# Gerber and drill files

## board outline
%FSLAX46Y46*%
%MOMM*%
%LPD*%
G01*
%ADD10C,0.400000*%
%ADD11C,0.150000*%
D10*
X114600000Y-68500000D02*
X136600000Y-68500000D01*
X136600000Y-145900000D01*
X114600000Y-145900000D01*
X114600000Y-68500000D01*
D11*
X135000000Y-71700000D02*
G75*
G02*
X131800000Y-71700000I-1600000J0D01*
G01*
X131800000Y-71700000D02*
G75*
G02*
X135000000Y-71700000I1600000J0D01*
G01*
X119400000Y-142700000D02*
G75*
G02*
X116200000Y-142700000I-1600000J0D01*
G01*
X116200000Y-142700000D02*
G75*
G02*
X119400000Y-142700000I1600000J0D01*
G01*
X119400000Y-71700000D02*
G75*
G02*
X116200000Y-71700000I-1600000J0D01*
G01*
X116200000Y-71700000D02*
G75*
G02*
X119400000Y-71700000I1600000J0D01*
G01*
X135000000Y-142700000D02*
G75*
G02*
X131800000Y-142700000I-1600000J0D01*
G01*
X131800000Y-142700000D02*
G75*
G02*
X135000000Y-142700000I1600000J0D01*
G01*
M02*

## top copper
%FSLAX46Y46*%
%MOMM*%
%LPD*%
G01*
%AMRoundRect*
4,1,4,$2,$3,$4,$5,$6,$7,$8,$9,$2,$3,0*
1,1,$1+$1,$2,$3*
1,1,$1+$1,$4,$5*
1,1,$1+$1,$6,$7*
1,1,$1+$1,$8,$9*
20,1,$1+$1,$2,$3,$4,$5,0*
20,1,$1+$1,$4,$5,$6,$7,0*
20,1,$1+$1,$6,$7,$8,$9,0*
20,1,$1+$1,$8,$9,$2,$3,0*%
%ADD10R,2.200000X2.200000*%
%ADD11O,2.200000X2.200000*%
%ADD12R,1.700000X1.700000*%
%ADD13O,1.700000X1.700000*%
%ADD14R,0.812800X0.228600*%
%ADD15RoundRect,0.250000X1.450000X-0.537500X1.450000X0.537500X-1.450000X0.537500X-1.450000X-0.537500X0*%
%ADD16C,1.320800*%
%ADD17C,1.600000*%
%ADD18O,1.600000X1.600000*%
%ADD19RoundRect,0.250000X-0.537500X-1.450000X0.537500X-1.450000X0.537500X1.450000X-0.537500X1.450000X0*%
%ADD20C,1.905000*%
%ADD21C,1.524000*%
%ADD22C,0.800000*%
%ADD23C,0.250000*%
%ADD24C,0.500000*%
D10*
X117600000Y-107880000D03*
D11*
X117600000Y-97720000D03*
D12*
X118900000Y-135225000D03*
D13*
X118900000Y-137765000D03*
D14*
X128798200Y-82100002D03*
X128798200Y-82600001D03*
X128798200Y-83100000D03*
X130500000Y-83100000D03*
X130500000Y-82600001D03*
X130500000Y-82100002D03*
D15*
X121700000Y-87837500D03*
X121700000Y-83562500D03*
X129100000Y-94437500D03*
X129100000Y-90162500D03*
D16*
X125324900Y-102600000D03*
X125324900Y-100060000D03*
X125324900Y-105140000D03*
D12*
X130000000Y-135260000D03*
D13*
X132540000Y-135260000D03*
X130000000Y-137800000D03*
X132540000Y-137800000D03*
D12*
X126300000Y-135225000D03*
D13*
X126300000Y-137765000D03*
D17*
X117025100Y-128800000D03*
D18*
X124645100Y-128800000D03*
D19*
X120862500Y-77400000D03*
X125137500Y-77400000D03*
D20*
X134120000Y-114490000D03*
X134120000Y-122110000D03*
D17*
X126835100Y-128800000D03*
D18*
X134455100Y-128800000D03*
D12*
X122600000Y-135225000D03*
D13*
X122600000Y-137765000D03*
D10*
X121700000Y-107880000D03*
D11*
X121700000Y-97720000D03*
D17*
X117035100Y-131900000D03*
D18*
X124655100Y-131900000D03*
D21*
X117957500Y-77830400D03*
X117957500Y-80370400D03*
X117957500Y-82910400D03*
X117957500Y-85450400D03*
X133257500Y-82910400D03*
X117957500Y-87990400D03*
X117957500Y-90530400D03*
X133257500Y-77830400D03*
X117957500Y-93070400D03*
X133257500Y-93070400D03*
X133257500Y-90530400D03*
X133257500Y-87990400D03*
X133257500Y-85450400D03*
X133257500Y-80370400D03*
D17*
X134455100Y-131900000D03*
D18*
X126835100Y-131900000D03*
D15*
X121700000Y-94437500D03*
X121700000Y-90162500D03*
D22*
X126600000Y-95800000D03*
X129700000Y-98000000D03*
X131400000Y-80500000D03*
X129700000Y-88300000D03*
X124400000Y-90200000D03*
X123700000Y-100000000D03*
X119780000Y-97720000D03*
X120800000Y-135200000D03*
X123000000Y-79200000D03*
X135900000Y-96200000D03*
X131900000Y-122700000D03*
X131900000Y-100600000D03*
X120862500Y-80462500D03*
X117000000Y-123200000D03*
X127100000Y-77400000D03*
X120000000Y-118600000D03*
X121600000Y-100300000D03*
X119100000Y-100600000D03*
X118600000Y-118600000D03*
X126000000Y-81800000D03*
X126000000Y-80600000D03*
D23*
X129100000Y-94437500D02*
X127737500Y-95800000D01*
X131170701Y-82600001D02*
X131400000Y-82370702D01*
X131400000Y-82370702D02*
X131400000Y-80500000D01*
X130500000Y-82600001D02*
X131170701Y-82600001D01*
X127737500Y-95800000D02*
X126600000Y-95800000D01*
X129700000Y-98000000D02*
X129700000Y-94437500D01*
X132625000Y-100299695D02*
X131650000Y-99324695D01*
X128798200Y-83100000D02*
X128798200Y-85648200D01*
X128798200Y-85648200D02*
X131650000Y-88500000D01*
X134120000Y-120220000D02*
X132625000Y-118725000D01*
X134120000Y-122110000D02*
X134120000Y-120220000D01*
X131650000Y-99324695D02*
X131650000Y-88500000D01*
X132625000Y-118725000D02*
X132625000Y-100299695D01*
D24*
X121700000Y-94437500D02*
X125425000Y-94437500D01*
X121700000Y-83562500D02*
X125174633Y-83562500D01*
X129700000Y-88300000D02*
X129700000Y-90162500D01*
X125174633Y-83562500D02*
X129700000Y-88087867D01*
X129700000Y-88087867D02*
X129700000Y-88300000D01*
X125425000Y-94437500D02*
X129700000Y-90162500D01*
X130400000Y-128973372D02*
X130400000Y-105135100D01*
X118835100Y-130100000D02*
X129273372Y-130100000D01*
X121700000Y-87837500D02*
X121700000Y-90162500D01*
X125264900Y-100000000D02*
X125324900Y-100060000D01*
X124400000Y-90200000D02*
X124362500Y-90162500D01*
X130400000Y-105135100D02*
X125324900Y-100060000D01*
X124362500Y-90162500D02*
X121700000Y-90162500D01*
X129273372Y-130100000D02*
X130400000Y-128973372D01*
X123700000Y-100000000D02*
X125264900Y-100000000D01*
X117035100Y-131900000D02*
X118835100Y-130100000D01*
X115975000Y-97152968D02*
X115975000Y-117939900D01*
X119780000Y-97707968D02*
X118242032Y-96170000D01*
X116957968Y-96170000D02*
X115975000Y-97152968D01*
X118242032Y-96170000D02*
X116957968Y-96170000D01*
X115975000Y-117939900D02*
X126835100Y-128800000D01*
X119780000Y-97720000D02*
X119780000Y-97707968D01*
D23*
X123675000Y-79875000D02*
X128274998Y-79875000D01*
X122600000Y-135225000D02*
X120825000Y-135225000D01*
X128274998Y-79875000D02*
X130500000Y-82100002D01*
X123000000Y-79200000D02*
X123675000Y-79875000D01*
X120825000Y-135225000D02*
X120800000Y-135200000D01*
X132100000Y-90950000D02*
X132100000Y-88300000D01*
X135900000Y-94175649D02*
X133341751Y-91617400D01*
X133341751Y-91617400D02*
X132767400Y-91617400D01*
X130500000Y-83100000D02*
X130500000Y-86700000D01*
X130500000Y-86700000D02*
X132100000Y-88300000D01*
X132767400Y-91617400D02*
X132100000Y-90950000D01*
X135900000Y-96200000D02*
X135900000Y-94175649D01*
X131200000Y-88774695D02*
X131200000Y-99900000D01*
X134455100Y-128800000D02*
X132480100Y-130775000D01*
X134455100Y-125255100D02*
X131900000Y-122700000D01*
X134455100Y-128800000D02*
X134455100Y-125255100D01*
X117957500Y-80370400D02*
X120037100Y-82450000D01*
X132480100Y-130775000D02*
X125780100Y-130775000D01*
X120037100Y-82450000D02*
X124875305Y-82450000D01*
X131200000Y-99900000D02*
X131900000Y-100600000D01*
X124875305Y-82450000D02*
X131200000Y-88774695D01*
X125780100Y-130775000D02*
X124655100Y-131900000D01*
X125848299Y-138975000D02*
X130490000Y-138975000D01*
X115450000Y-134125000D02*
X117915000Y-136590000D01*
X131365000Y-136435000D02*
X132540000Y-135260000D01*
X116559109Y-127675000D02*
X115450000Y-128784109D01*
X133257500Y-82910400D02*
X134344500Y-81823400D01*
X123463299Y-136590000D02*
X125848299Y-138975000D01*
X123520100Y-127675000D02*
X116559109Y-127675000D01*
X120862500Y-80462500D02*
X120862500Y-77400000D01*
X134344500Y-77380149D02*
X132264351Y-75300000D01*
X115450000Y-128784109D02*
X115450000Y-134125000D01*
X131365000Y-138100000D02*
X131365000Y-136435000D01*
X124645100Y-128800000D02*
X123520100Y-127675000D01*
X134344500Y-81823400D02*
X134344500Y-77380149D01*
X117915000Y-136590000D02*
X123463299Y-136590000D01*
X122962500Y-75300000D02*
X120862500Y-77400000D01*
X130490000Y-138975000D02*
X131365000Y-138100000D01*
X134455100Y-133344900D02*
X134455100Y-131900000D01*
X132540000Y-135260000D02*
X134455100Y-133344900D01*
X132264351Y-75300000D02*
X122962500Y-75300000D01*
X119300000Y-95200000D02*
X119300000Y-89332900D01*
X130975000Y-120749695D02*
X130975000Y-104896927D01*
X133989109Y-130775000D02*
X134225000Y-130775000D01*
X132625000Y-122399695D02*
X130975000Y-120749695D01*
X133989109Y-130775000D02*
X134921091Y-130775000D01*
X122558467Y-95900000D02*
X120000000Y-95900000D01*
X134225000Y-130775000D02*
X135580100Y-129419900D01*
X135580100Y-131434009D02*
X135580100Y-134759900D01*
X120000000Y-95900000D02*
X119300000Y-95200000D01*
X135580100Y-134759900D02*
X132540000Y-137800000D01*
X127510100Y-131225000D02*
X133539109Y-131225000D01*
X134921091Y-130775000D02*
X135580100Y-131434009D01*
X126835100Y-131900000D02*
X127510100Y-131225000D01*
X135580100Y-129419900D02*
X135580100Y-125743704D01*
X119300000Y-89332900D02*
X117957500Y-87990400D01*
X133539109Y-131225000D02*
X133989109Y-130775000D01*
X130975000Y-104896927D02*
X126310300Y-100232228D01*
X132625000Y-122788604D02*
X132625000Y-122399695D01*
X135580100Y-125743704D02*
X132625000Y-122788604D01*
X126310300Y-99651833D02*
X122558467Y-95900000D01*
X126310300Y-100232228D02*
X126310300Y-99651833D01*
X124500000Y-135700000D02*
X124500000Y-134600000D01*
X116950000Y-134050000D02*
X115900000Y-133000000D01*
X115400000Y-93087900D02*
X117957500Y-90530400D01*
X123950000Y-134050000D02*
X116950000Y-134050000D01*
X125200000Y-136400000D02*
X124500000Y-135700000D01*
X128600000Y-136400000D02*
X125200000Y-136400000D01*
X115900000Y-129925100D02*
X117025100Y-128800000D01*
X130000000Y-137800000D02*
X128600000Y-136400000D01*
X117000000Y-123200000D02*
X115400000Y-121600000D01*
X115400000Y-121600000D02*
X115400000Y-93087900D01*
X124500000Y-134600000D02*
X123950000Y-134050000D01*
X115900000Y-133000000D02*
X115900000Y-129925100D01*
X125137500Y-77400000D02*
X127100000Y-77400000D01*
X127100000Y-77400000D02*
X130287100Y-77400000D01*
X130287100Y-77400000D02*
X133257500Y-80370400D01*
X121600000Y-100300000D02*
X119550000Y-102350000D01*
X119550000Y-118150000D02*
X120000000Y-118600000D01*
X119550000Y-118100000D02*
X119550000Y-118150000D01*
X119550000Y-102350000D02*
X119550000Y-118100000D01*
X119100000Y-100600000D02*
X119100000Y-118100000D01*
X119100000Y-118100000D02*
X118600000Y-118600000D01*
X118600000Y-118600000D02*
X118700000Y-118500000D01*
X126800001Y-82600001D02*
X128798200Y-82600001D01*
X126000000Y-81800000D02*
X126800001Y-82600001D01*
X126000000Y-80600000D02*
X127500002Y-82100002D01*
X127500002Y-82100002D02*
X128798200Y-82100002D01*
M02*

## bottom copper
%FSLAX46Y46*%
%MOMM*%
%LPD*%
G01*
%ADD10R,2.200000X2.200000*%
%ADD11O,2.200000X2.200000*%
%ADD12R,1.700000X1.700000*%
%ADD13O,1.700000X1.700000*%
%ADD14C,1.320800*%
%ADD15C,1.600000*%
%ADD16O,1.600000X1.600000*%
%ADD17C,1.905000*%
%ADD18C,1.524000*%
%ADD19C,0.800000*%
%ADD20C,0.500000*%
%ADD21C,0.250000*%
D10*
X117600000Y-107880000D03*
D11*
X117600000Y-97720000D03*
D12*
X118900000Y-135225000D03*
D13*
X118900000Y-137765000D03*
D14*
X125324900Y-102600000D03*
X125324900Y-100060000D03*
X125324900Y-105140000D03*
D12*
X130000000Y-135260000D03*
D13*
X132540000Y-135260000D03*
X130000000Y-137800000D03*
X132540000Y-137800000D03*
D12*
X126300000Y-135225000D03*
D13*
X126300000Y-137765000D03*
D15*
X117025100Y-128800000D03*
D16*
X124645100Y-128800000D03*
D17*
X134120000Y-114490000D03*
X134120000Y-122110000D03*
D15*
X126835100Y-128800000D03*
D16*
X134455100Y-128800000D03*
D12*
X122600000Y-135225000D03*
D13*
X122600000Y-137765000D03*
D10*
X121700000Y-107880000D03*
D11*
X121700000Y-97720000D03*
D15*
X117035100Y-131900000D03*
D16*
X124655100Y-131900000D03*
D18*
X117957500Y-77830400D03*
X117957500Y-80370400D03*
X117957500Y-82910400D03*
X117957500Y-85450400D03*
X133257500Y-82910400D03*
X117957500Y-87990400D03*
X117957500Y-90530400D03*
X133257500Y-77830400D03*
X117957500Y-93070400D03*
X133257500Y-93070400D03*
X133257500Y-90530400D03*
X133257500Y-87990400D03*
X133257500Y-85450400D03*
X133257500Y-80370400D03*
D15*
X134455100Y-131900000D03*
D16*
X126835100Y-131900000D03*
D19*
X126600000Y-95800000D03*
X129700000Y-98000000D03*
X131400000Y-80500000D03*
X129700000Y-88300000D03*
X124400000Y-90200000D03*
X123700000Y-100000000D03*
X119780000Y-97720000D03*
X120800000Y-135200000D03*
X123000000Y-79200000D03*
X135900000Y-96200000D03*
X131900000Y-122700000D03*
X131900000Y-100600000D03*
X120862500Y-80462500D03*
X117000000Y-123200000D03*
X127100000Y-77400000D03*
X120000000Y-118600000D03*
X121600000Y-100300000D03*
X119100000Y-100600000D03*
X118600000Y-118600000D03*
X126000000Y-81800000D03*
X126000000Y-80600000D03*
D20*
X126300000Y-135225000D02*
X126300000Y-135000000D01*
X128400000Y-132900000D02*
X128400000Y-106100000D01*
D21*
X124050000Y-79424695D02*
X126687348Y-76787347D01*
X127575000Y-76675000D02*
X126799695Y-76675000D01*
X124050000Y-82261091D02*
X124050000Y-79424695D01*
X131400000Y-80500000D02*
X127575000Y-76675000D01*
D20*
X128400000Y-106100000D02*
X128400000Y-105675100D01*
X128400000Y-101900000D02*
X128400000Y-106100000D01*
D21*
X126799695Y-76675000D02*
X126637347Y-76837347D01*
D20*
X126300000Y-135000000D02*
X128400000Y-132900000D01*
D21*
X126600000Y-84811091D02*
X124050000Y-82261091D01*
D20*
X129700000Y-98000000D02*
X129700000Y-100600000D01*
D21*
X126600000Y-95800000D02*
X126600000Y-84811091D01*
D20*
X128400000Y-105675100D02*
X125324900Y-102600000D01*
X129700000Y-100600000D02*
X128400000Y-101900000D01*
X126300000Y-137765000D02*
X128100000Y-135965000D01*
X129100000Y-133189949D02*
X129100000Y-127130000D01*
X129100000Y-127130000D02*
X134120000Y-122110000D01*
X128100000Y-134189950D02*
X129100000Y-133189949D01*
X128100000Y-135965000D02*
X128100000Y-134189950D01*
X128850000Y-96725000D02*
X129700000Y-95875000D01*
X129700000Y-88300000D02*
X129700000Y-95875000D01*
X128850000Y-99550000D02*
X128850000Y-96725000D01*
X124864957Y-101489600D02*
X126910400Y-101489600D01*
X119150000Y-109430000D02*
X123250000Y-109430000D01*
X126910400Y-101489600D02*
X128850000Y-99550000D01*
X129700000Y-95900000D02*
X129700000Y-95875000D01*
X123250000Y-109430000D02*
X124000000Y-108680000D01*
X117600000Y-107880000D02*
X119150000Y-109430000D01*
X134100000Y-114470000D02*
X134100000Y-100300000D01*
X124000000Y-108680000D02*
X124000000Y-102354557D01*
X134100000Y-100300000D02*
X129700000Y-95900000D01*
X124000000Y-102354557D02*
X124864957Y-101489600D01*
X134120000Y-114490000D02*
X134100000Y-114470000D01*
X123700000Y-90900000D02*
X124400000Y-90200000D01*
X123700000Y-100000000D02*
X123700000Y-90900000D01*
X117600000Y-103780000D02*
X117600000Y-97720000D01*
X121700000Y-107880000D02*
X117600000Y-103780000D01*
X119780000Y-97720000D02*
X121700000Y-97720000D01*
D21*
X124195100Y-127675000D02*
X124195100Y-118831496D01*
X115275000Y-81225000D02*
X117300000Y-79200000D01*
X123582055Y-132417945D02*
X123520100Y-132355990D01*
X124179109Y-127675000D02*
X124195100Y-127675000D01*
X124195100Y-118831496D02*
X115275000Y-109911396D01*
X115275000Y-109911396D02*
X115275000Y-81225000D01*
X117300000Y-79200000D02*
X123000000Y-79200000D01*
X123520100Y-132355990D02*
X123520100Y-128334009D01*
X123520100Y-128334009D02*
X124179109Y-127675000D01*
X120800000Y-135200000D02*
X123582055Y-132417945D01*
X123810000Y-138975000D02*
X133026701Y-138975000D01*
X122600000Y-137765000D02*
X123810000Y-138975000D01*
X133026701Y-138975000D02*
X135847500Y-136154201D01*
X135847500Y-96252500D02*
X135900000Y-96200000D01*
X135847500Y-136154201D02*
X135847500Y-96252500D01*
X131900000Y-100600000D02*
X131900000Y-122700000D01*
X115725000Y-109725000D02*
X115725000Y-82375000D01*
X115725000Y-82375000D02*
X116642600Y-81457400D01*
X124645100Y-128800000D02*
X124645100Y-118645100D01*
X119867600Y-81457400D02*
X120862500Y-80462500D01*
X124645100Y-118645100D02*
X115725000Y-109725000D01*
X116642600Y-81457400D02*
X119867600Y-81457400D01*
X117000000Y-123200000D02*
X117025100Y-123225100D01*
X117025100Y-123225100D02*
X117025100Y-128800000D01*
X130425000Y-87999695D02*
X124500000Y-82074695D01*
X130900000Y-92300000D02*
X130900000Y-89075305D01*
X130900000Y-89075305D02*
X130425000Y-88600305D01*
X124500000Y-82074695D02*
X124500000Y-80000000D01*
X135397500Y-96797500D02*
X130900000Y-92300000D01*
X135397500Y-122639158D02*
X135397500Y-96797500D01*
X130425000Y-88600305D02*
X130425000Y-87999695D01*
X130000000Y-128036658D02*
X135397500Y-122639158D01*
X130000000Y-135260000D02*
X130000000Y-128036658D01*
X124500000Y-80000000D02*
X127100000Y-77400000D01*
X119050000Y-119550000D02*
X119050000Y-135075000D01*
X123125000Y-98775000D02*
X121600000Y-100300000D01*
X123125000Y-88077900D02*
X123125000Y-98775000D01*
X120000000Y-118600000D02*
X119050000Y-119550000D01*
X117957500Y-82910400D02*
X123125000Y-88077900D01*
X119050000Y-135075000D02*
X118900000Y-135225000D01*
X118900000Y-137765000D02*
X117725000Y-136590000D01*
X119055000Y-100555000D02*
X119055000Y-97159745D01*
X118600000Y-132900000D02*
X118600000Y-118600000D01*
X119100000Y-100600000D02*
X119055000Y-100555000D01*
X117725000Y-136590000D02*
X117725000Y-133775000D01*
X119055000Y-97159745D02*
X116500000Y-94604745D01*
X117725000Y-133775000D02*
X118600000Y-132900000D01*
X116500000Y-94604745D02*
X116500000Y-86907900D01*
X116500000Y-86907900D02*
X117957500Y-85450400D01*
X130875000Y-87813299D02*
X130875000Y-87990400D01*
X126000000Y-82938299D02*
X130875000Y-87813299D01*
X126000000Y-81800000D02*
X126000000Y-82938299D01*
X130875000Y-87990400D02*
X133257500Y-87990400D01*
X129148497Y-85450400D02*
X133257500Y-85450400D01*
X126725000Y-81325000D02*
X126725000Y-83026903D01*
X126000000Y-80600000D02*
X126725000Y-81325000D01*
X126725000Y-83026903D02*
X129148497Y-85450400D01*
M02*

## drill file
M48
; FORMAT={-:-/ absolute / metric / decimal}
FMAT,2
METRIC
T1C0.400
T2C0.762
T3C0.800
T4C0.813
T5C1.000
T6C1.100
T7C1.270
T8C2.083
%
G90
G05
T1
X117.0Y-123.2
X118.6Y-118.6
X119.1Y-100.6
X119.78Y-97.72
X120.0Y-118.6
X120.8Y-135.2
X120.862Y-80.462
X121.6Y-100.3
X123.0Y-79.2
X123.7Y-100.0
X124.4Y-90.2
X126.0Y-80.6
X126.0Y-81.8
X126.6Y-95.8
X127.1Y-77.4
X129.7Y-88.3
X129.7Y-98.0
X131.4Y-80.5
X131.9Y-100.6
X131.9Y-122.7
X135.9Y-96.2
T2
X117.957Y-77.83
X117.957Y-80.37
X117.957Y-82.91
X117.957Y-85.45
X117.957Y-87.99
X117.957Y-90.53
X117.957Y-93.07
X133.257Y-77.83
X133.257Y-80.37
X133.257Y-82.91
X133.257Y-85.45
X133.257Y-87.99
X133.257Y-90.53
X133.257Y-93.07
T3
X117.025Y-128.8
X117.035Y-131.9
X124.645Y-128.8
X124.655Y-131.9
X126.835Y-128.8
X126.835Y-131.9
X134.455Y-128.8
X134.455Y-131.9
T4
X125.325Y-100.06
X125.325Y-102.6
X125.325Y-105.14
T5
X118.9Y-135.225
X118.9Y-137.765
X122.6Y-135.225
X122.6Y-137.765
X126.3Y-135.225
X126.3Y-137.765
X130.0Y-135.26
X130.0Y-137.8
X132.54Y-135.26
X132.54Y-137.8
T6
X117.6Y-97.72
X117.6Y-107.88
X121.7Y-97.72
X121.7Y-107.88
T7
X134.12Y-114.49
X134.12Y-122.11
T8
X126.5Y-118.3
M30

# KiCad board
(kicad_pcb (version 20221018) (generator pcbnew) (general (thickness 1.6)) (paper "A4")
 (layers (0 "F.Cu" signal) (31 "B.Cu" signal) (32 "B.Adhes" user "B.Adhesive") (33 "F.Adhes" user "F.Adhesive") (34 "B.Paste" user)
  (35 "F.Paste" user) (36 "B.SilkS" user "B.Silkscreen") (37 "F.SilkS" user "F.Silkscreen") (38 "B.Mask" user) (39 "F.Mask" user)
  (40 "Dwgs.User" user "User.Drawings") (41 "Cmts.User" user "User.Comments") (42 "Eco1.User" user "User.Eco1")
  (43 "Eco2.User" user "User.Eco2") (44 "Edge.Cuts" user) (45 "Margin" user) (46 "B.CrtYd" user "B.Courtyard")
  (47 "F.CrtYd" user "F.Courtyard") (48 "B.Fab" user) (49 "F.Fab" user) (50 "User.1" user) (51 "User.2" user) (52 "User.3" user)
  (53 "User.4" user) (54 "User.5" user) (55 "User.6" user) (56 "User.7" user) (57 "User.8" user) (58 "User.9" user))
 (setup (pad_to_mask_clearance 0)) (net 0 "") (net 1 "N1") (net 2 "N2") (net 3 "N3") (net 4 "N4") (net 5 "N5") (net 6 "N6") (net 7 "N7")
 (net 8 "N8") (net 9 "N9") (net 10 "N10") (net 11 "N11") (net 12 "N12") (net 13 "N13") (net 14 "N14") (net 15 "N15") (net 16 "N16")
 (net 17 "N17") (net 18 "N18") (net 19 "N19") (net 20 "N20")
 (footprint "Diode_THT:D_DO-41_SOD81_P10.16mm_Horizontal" (layer "F.Cu") (at 117.6 107.88 90)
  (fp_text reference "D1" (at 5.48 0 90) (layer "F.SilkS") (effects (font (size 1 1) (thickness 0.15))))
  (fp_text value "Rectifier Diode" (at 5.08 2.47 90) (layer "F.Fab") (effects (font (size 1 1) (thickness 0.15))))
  (pad "1" thru_hole rect (at 0 0 90) (size 2.2 2.2) (drill 1.1) (layers "*.Cu" "*.Mask") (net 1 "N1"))
  (pad "2" thru_hole oval (at 10.16 0 90) (size 2.2 2.2) (drill 1.1) (layers "*.Cu" "*.Mask") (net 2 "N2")))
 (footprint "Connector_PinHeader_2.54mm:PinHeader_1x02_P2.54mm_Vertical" (layer "F.Cu") (at 118.9 135.225)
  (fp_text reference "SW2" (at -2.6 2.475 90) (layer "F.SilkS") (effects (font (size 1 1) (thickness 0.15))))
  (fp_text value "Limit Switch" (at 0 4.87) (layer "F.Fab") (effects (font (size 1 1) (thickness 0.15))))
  (pad "1" thru_hole rect (at 0 0) (size 1.7 1.7) (drill 1) (layers "*.Cu" "*.Mask") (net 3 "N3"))
  (pad "2" thru_hole oval (at 0 2.54) (size 1.7 1.7) (drill 1) (layers "*.Cu" "*.Mask") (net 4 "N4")))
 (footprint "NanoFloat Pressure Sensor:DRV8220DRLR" (layer "F.Cu") (at 129.6491 82.600001)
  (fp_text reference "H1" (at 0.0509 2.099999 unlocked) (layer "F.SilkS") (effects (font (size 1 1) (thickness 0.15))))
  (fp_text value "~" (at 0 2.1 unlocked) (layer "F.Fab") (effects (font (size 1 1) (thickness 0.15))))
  (pad "1" smd rect (at -0.8509 -0.499999) (size 0.8128 0.2286) (layers "F.Cu" "F.Paste" "F.Mask") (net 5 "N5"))
  (pad "2" smd rect (at -0.8509 0) (size 0.8128 0.2286) (layers "F.Cu" "F.Paste" "F.Mask") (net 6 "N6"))
  (pad "3" smd rect (at -0.8509 0.499999) (size 0.8128 0.2286) (layers "F.Cu" "F.Paste" "F.Mask") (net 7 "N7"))
  (pad "4" smd rect (at 0.8509 0.499999) (size 0.8128 0.2286) (layers "F.Cu" "F.Paste" "F.Mask") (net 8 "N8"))
  (pad "5" smd rect (at 0.8509 0) (size 0.8128 0.2286) (layers "F.Cu" "F.Paste" "F.Mask") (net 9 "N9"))
  (pad "6" smd rect (at 0.8509 -0.499999) (size 0.8128 0.2286) (layers "F.Cu" "F.Paste" "F.Mask") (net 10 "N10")))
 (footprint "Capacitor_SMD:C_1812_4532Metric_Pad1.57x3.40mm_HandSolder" (layer "F.Cu") (at 121.7 85.7 90)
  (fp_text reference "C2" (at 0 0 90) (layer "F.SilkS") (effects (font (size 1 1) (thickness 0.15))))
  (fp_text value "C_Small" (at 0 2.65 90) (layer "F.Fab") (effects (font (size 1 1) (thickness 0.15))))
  (pad "1" smd roundrect (at -2.1375 0 90) (size 1.575 3.4) (layers "F.Cu" "F.Paste" "F.Mask") (roundrect_rratio 0.1587301587)
   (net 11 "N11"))
  (pad "2" smd roundrect (at 2.1375 0 90) (size 1.575 3.4) (layers "F.Cu" "F.Paste" "F.Mask") (roundrect_rratio 0.1587301587) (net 1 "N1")))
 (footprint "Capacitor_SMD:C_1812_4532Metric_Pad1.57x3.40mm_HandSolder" (layer "F.Cu") (at 129.1 92.3 90)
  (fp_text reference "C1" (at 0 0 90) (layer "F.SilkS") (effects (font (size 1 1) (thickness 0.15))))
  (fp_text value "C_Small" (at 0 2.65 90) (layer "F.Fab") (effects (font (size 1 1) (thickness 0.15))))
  (pad "1" smd roundrect (at -2.1375 0 90) (size 1.575 3.4) (layers "F.Cu" "F.Paste" "F.Mask") (roundrect_rratio 0.1587301587) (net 9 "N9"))
  (pad "2" smd roundrect (at 2.1375 0 90) (size 1.575 3.4) (layers "F.Cu" "F.Paste" "F.Mask") (roundrect_rratio 0.1587301587) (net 1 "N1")))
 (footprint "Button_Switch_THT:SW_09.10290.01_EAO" (layer "F.Cu") (at 125.3249 102.6 90)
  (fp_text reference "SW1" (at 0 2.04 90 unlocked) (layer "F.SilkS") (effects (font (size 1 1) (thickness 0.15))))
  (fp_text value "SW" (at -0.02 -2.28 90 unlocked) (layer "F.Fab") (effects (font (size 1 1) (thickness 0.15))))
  (pad "1" thru_hole circle (at 0 0 90) (size 1.3208 1.3208) (drill 0.8128) (layers "*.Cu" "*.Mask") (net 9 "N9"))
  (pad "2" thru_hole circle (at 2.54 0 90) (size 1.3208 1.3208) (drill 0.8128) (layers "*.Cu" "*.Mask") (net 11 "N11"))
  (pad "3" thru_hole circle (at -2.54 0 90) (size 1.3208 1.3208) (drill 0.8128) (layers "*.Cu" "*.Mask") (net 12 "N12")))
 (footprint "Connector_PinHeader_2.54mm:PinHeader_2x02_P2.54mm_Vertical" (layer "F.Cu") (at 130 135.26)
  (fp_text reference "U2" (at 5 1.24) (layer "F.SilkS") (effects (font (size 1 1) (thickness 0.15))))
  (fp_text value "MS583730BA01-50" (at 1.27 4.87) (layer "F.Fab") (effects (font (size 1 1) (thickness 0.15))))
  (pad "1" thru_hole rect (at 0 0) (size 1.7 1.7) (drill 1) (layers "*.Cu" "*.Mask") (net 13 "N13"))
  (pad "2" thru_hole oval (at 2.54 0) (size 1.7 1.7) (drill 1) (layers "*.Cu" "*.Mask") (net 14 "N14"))
  (pad "3" thru_hole oval (at 0 2.54) (size 1.7 1.7) (drill 1) (layers "*.Cu" "*.Mask") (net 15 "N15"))
  (pad "4" thru_hole oval (at 2.54 2.54) (size 1.7 1.7) (drill 1) (layers "*.Cu" "*.Mask") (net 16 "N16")))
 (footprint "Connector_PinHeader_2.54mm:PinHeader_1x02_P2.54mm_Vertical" (layer "F.Cu") (at 126.3 135.225)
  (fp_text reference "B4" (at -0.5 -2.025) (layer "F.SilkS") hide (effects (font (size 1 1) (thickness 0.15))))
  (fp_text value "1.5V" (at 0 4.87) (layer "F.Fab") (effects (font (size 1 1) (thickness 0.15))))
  (pad "1" thru_hole rect (at 0 0) (size 1.7 1.7) (drill 1) (layers "*.Cu" "*.Mask") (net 9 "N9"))
  (pad "2" thru_hole oval (at 0 2.54) (size 1.7 1.7) (drill 1) (layers "*.Cu" "*.Mask") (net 7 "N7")))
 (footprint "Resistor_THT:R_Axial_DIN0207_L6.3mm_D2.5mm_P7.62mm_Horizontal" (layer "F.Cu") (at 117.0251 128.8)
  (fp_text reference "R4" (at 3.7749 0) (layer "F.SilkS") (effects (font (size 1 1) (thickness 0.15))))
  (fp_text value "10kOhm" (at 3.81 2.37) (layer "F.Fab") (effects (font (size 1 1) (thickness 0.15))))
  (pad "1" thru_hole circle (at 0 0) (size 1.6 1.6) (drill 0.8) (layers "*.Cu" "*.Mask") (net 15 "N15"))
  (pad "2" thru_hole oval (at 7.62 0) (size 1.6 1.6) (drill 0.8) (layers "*.Cu" "*.Mask") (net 14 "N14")))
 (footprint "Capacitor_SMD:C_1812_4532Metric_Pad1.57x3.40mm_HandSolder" (layer "F.Cu") (at 123 77.4)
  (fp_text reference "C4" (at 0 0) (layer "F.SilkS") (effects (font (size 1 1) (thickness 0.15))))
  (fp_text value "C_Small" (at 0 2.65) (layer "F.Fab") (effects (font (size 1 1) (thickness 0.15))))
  (pad "1" smd roundrect (at -2.1375 0) (size 1.575 3.4) (layers "F.Cu" "F.Paste" "F.Mask") (roundrect_rratio 0.1587301587) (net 14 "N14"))
  (pad "2" smd roundrect (at 2.1375 0) (size 1.575 3.4) (layers "F.Cu" "F.Paste" "F.Mask") (roundrect_rratio 0.1587301587) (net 13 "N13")))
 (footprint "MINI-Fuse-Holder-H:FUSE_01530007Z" (layer "F.Cu") (at 126.5 118.3 -90)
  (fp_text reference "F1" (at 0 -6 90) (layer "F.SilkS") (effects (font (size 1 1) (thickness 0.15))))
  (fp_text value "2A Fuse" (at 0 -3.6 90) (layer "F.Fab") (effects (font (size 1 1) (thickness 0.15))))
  (pad "" np_thru_hole circle (at 0 0 270) (size 2.0828 2.0828) (drill 2.0828) (layers "*.Cu" "*.Mask"))
  (pad "1" thru_hole circle (at -3.81 -7.62 270) (size 1.905 1.905) (drill 1.27) (layers "*.Cu" "*.Mask") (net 1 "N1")
   (solder_mask_margin 0.102))
  (pad "2" thru_hole circle (at 3.81 -7.62 270) (size 1.905 1.905) (drill 1.27) (layers "*.Cu" "*.Mask") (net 7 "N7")
   (solder_mask_margin 0.102)))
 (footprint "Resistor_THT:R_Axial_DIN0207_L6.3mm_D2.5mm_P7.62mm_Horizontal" (layer "F.Cu") (at 126.8351 128.8)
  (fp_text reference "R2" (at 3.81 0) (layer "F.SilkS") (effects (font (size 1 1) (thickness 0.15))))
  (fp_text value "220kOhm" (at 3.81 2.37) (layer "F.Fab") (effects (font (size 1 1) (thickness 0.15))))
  (pad "1" thru_hole circle (at 0 0) (size 1.6 1.6) (drill 0.8) (layers "*.Cu" "*.Mask") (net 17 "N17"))
  (pad "2" thru_hole oval (at 7.62 0) (size 1.6 1.6) (drill 0.8) (layers "*.Cu" "*.Mask") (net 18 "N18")))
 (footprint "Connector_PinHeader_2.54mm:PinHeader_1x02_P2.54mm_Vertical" (layer "F.Cu") (at 122.6 135.225)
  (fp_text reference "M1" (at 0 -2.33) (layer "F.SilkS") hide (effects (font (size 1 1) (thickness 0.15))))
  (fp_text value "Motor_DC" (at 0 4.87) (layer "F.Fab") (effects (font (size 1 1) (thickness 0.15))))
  (pad "1" thru_hole rect (at 0 0) (size 1.7 1.7) (drill 1) (layers "*.Cu" "*.Mask") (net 10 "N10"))
  (pad "2" thru_hole oval (at 0 2.54) (size 1.7 1.7) (drill 1) (layers "*.Cu" "*.Mask") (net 8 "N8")))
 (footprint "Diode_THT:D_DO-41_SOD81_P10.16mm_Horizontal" (layer "F.Cu") (at 121.7 107.88 90)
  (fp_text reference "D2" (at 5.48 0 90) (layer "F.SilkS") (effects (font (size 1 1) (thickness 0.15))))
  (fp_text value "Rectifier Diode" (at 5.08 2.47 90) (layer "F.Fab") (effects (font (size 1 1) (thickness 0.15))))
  (pad "1" thru_hole rect (at 0 0 90) (size 2.2 2.2) (drill 1.1) (layers "*.Cu" "*.Mask") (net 2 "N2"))
  (pad "2" thru_hole oval (at 10.16 0 90) (size 2.2 2.2) (drill 1.1) (layers "*.Cu" "*.Mask") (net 17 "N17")))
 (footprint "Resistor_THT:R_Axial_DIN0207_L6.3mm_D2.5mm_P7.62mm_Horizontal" (layer "F.Cu") (at 117.0351 131.9)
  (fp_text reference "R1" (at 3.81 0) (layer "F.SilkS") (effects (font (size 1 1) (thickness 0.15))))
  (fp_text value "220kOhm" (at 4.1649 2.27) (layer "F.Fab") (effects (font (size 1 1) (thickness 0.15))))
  (pad "1" thru_hole circle (at 0 0) (size 1.6 1.6) (drill 0.8) (layers "*.Cu" "*.Mask") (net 11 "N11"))
  (pad "2" thru_hole oval (at 7.62 0) (size 1.6 1.6) (drill 0.8) (layers "*.Cu" "*.Mask") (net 18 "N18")))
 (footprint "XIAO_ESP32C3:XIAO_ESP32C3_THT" (layer "F.Cu") (at 125.5575 87.8704)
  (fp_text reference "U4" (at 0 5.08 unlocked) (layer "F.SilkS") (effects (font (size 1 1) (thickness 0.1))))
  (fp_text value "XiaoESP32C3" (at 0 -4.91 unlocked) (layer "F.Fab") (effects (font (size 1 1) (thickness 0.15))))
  (pad "0" thru_hole circle (at -7.6 -10.04) (size 1.524 1.524) (drill 0.762) (layers "*.Cu" "*.Mask"))
  (pad "1" thru_hole circle (at -7.6 -7.5) (size 1.524 1.524) (drill 0.762) (layers "*.Cu" "*.Mask") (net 18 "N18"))
  (pad "2" thru_hole circle (at -7.6 -4.96) (size 1.524 1.524) (drill 0.762) (layers "*.Cu" "*.Mask") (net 3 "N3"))
  (pad "3" thru_hole circle (at -7.6 -2.42) (size 1.524 1.524) (drill 0.762) (layers "*.Cu" "*.Mask") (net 4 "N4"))
  (pad "3V3" thru_hole circle (at 7.7 -4.96) (size 1.524 1.524) (drill 0.762) (layers "*.Cu" "*.Mask") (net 14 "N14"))
  (pad "4" thru_hole circle (at -7.6 0.12) (size 1.524 1.524) (drill 0.762) (layers "*.Cu" "*.Mask") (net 16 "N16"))
  (pad "5" thru_hole circle (at -7.6 2.66) (size 1.524 1.524) (drill 0.762) (layers "*.Cu" "*.Mask") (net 15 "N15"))
  (pad "5V" thru_hole circle (at 7.7 -10.04) (size 1.524 1.524) (drill 0.762) (layers "*.Cu" "*.Mask"))
  (pad "6" thru_hole circle (at -7.6 5.2) (size 1.524 1.524) (drill 0.762) (layers "*.Cu" "*.Mask"))
  (pad "7" thru_hole circle (at 7.7 5.2) (size 1.524 1.524) (drill 0.762) (layers "*.Cu" "*.Mask") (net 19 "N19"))
  (pad "8" thru_hole circle (at 7.7 2.66) (size 1.524 1.524) (drill 0.762) (layers "*.Cu" "*.Mask") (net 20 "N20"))
  (pad "9" thru_hole circle (at 7.7 0.12) (size 1.524 1.524) (drill 0.762) (layers "*.Cu" "*.Mask") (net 6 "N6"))
  (pad "10" thru_hole circle (at 7.7 -2.42) (size 1.524 1.524) (drill 0.762) (layers "*.Cu" "*.Mask") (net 5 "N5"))
  (pad "GND" thru_hole circle (at 7.7 -7.5) (size 1.524 1.524) (drill 0.762) (layers "*.Cu" "*.Mask") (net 13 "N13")))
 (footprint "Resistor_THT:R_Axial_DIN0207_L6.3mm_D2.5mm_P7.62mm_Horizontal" (layer "F.Cu") (at 134.4551 131.9 180)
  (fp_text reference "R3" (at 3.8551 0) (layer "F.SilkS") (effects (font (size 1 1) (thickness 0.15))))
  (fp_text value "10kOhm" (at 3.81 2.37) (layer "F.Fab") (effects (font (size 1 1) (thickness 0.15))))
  (pad "1" thru_hole circle (at 0 0 180) (size 1.6 1.6) (drill 0.8) (layers "*.Cu" "*.Mask") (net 14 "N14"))
  (pad "2" thru_hole oval (at 7.62 0 180) (size 1.6 1.6) (drill 0.8) (layers "*.Cu" "*.Mask") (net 16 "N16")))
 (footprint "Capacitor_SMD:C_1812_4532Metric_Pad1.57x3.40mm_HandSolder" (layer "F.Cu") (at 121.7 92.3 90)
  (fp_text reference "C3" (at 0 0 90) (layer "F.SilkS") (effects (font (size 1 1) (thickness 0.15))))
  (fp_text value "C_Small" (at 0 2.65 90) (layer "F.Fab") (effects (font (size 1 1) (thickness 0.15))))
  (pad "1" smd roundrect (at -2.1375 0 90) (size 1.575 3.4) (layers "F.Cu" "F.Paste" "F.Mask") (roundrect_rratio 0.1587301587) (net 1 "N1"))
  (pad "2" smd roundrect (at 2.1375 0 90) (size 1.575 3.4) (layers "F.Cu" "F.Paste" "F.Mask") (roundrect_rratio 0.1587301587) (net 11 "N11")))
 (gr_rect (start 114.6 68.5) (end 136.6 145.9) (stroke (width 0.4) (type default)) (fill none) (layer "Edge.Cuts"))
 (gr_circle (center 133.4 71.7) (end 135 71.7) (stroke (width 0.15) (type default)) (fill none) (layer "Edge.Cuts"))
 (gr_circle (center 117.8 142.7) (end 119.4 142.7) (stroke (width 0.15) (type default)) (fill none) (layer "Edge.Cuts"))
 (gr_circle (center 117.8 71.7) (end 119.4 71.7) (stroke (width 0.15) (type default)) (fill none) (layer "Edge.Cuts"))
 (gr_circle (center 133.4 142.7) (end 135 142.7) (stroke (width 0.15) (type default)) (fill none) (layer "Edge.Cuts"))
 (segment (start 129.1 94.4375) (end 127.7375 95.8) (width 0.25) (layer "F.Cu") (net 9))
 (segment (start 131.170701 82.600001) (end 131.4 82.370702) (width 0.25) (layer "F.Cu") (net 9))
 (segment (start 131.4 82.370702) (end 131.4 80.5) (width 0.25) (layer "F.Cu") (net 9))
 (segment (start 130.5 82.600001) (end 131.170701 82.600001) (width 0.25) (layer "F.Cu") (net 9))
 (segment (start 127.7375 95.8) (end 126.6 95.8) (width 0.25) (layer "F.Cu") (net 9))
 (segment (start 129.7 98) (end 129.7 94.4375) (width 0.25) (layer "F.Cu") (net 9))
 (via (at 126.6 95.8) (size 0.8) (drill 0.4) (layers "F.Cu" "B.Cu") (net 9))
 (via (at 129.7 98) (size 0.8) (drill 0.4) (layers "F.Cu" "B.Cu") (free) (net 9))
 (via (at 131.4 80.5) (size 0.8) (drill 0.4) (layers "F.Cu" "B.Cu") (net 9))
 (segment (start 126.3 135.225) (end 126.3 135) (width 0.5) (layer "B.Cu") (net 9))
 (segment (start 128.4 132.9) (end 128.4 106.1) (width 0.5) (layer "B.Cu") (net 9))
 (segment (start 124.05 79.424695) (end 126.687348 76.787347) (width 0.25) (layer "B.Cu") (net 9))
 (segment (start 127.575 76.675) (end 126.799695 76.675) (width 0.25) (layer "B.Cu") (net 9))
 (segment (start 124.05 82.261091) (end 124.05 79.424695) (width 0.25) (layer "B.Cu") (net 9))
 (segment (start 131.4 80.5) (end 127.575 76.675) (width 0.25) (layer "B.Cu") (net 9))
 (segment (start 128.4 106.1) (end 128.4 105.6751) (width 0.5) (layer "B.Cu") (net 9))
 (segment (start 128.4 101.9) (end 128.4 106.1) (width 0.5) (layer "B.Cu") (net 9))
 (segment (start 126.799695 76.675) (end 126.637347 76.837347) (width 0.25) (layer "B.Cu") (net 9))
 (segment (start 126.3 135) (end 128.4 132.9) (width 0.5) (layer "B.Cu") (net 9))
 (segment (start 126.6 84.811091) (end 124.05 82.261091) (width 0.25) (layer "B.Cu") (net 9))
 (segment (start 129.7 98) (end 129.7 100.6) (width 0.5) (layer "B.Cu") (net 9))
 (segment (start 126.6 95.8) (end 126.6 84.811091) (width 0.25) (layer "B.Cu") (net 9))
 (segment (start 128.4 105.6751) (end 125.3249 102.6) (width 0.5) (layer "B.Cu") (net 9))
 (segment (start 129.7 100.6) (end 128.4 101.9) (width 0.5) (layer "B.Cu") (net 9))
 (segment (start 132.625 100.299695) (end 131.65 99.324695) (width 0.25) (layer "F.Cu") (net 7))
 (segment (start 128.7982 83.1) (end 128.7982 85.6482) (width 0.25) (layer "F.Cu") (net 7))
 (segment (start 128.7982 85.6482) (end 131.65 88.5) (width 0.25) (layer "F.Cu") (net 7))
 (segment (start 134.12 120.22) (end 132.625 118.725) (width 0.25) (layer "F.Cu") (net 7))
 (segment (start 134.12 122.11) (end 134.12 120.22) (width 0.25) (layer "F.Cu") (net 7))
 (segment (start 131.65 99.324695) (end 131.65 88.5) (width 0.25) (layer "F.Cu") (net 7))
 (segment (start 132.625 118.725) (end 132.625 100.299695) (width 0.25) (layer "F.Cu") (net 7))
 (segment (start 126.3 137.765) (end 128.1 135.965) (width 0.5) (layer "B.Cu") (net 7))
 (segment (start 129.1 133.189949) (end 129.1 127.13) (width 0.5) (layer "B.Cu") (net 7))
 (segment (start 129.1 127.13) (end 134.12 122.11) (width 0.5) (layer "B.Cu") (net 7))
 (segment (start 128.1 134.18995) (end 129.1 133.189949) (width 0.5) (layer "B.Cu") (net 7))
 (segment (start 128.1 135.965) (end 128.1 134.18995) (width 0.5) (layer "B.Cu") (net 7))
 (segment (start 121.7 94.4375) (end 125.425 94.4375) (width 0.5) (layer "F.Cu") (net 1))
 (segment (start 121.7 83.5625) (end 125.174633 83.5625) (width 0.5) (layer "F.Cu") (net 1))
 (segment (start 129.7 88.3) (end 129.7 90.1625) (width 0.5) (layer "F.Cu") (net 1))
 (segment (start 125.174633 83.5625) (end 129.7 88.087867) (width 0.5) (layer "F.Cu") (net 1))
 (segment (start 129.7 88.087867) (end 129.7 88.3) (width 0.5) (layer "F.Cu") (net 1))
 (segment (start 125.425 94.4375) (end 129.7 90.1625) (width 0.5) (layer "F.Cu") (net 1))
 (via (at 129.7 88.3) (size 0.8) (drill 0.4) (layers "F.Cu" "B.Cu") (free) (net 1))
 (segment (start 128.85 96.725) (end 129.7 95.875) (width 0.5) (layer "B.Cu") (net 1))
 (segment (start 129.7 88.3) (end 129.7 95.875) (width 0.5) (layer "B.Cu") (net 1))
 (segment (start 128.85 99.55) (end 128.85 96.725) (width 0.5) (layer "B.Cu") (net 1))
 (segment (start 124.864957 101.4896) (end 126.9104 101.4896) (width 0.5) (layer "B.Cu") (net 1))
 (segment (start 119.15 109.43) (end 123.25 109.43) (width 0.5) (layer "B.Cu") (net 1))
 (segment (start 126.9104 101.4896) (end 128.85 99.55) (width 0.5) (layer "B.Cu") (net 1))
 (segment (start 129.7 95.9) (end 129.7 95.875) (width 0.5) (layer "B.Cu") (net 1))
 (segment (start 123.25 109.43) (end 124 108.68) (width 0.5) (layer "B.Cu") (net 1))
 (segment (start 117.6 107.88) (end 119.15 109.43) (width 0.5) (layer "B.Cu") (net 1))
 (segment (start 134.1 114.47) (end 134.1 100.3) (width 0.5) (layer "B.Cu") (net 1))
 (segment (start 124 108.68) (end 124 102.354557) (width 0.5) (layer "B.Cu") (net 1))
 (segment (start 134.1 100.3) (end 129.7 95.9) (width 0.5) (layer "B.Cu") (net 1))
 (segment (start 124 102.354557) (end 124.864957 101.4896) (width 0.5) (layer "B.Cu") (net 1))
 (segment (start 134.12 114.49) (end 134.1 114.47) (width 0.5) (layer "B.Cu") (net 1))
 (segment (start 130.4 128.973372) (end 130.4 105.1351) (width 0.5) (layer "F.Cu") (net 11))
 (segment (start 118.8351 130.1) (end 129.273372 130.1) (width 0.5) (layer "F.Cu") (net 11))
 (segment (start 121.7 87.8375) (end 121.7 90.1625) (width 0.5) (layer "F.Cu") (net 11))
 (segment (start 125.2649 100) (end 125.3249 100.06) (width 0.5) (layer "F.Cu") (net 11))
 (segment (start 124.4 90.2) (end 124.3625 90.1625) (width 0.5) (layer "F.Cu") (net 11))
 (segment (start 130.4 105.1351) (end 125.3249 100.06) (width 0.5) (layer "F.Cu") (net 11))
 (segment (start 124.3625 90.1625) (end 121.7 90.1625) (width 0.5) (layer "F.Cu") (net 11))
 (segment (start 129.273372 130.1) (end 130.4 128.973372) (width 0.5) (layer "F.Cu") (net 11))
 (segment (start 123.7 100) (end 125.2649 100) (width 0.5) (layer "F.Cu") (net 11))
 (segment (start 117.0351 131.9) (end 118.8351 130.1) (width 0.5) (layer "F.Cu") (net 11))
 (via (at 124.4 90.2) (size 0.8) (drill 0.4) (layers "F.Cu" "B.Cu") (free) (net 11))
 (via (at 123.7 100) (size 0.8) (drill 0.4) (layers "F.Cu" "B.Cu") (free) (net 11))
 (segment (start 123.7 90.9) (end 124.4 90.2) (width 0.5) (layer "B.Cu") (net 11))
 (segment (start 123.7 100) (end 123.7 90.9) (width 0.5) (layer "B.Cu") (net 11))
 (segment (start 117.6 103.78) (end 117.6 97.72) (width 0.5) (layer "B.Cu") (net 2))
 (segment (start 121.7 107.88) (end 117.6 103.78) (width 0.5) (layer "B.Cu") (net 2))
 (segment (start 115.975 97.152968) (end 115.975 117.9399) (width 0.5) (layer "F.Cu") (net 17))
 (segment (start 119.78 97.707968) (end 118.242032 96.17) (width 0.5) (layer "F.Cu") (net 17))
 (segment (start 116.957968 96.17) (end 115.975 97.152968) (width 0.5) (layer "F.Cu") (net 17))
 (segment (start 118.242032 96.17) (end 116.957968 96.17) (width 0.5) (layer "F.Cu") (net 17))
 (segment (start 115.975 117.9399) (end 126.8351 128.8) (width 0.5) (layer "F.Cu") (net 17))
 (segment (start 119.78 97.72) (end 119.78 97.707968) (width 0.5) (layer "F.Cu") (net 17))
 (via (at 119.78 97.72) (size 0.8) (drill 0.4) (layers "F.Cu" "B.Cu") (free) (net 17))
 (segment (start 119.78 97.72) (end 121.7 97.72) (width 0.5) (layer "B.Cu") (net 17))
 (segment (start 123.675 79.875) (end 128.274998 79.875) (width 0.25) (layer "F.Cu") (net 10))
 (segment (start 122.6 135.225) (end 120.825 135.225) (width 0.25) (layer "F.Cu") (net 10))
 (segment (start 128.274998 79.875) (end 130.5 82.100002) (width 0.25) (layer "F.Cu") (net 10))
 (segment (start 123 79.2) (end 123.675 79.875) (width 0.25) (layer "F.Cu") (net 10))
 (segment (start 120.825 135.225) (end 120.8 135.2) (width 0.25) (layer "F.Cu") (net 10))
 (via (at 120.8 135.2) (size 0.8) (drill 0.4) (layers "F.Cu" "B.Cu") (free) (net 10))
 (via (at 123 79.2) (size 0.8) (drill 0.4) (layers "F.Cu" "B.Cu") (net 10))
 (segment (start 124.1951 127.675) (end 124.1951 118.831496) (width 0.25) (layer "B.Cu") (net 10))
 (segment (start 115.275 81.225) (end 117.3 79.2) (width 0.25) (layer "B.Cu") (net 10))
 (segment (start 123.582055 132.417945) (end 123.5201 132.35599) (width 0.25) (layer "B.Cu") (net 10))
 (segment (start 124.179109 127.675) (end 124.1951 127.675) (width 0.25) (layer "B.Cu") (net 10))
 (segment (start 124.1951 118.831496) (end 115.275 109.911396) (width 0.25) (layer "B.Cu") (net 10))
 (segment (start 115.275 109.911396) (end 115.275 81.225) (width 0.25) (layer "B.Cu") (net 10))
 (segment (start 117.3 79.2) (end 123 79.2) (width 0.25) (layer "B.Cu") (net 10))
 (segment (start 123.5201 132.35599) (end 123.5201 128.334009) (width 0.25) (layer "B.Cu") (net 10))
 (segment (start 123.5201 128.334009) (end 124.179109 127.675) (width 0.25) (layer "B.Cu") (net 10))
 (segment (start 120.8 135.2) (end 123.582055 132.417945) (width 0.25) (layer "B.Cu") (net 10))
 (segment (start 132.1 90.95) (end 132.1 88.3) (width 0.25) (layer "F.Cu") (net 8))
 (segment (start 135.9 94.175649) (end 133.341751 91.6174) (width 0.25) (layer "F.Cu") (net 8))
 (segment (start 133.341751 91.6174) (end 132.7674 91.6174) (width 0.25) (layer "F.Cu") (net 8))
 (segment (start 130.5 83.1) (end 130.5 86.7) (width 0.25) (layer "F.Cu") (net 8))
 (segment (start 130.5 86.7) (end 132.1 88.3) (width 0.25) (layer "F.Cu") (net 8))
 (segment (start 132.7674 91.6174) (end 132.1 90.95) (width 0.25) (layer "F.Cu") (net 8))
 (segment (start 135.9 96.2) (end 135.9 94.175649) (width 0.25) (layer "F.Cu") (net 8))
 (via (at 135.9 96.2) (size 0.8) (drill 0.4) (layers "F.Cu" "B.Cu") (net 8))
 (segment (start 123.81 138.975) (end 133.026701 138.975) (width 0.25) (layer "B.Cu") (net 8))
 (segment (start 122.6 137.765) (end 123.81 138.975) (width 0.25) (layer "B.Cu") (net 8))
 (segment (start 133.026701 138.975) (end 135.8475 136.154201) (width 0.25) (layer "B.Cu") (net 8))
 (segment (start 135.8475 96.2525) (end 135.9 96.2) (width 0.25) (layer "B.Cu") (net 8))
 (segment (start 135.8475 136.154201) (end 135.8475 96.2525) (width 0.25) (layer "B.Cu") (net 8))
 (segment (start 131.2 88.774695) (end 131.2 99.9) (width 0.25) (layer "F.Cu") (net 18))
 (segment (start 134.4551 128.8) (end 132.4801 130.775) (width 0.25) (layer "F.Cu") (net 18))
 (segment (start 134.4551 125.2551) (end 131.9 122.7) (width 0.25) (layer "F.Cu") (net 18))
 (segment (start 134.4551 128.8) (end 134.4551 125.2551) (width 0.25) (layer "F.Cu") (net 18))
 (segment (start 117.9575 80.3704) (end 120.0371 82.45) (width 0.25) (layer "F.Cu") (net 18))
 (segment (start 132.4801 130.775) (end 125.7801 130.775) (width 0.25) (layer "F.Cu") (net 18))
 (segment (start 120.0371 82.45) (end 124.875305 82.45) (width 0.25) (layer "F.Cu") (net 18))
 (segment (start 131.2 99.9) (end 131.9 100.6) (width 0.25) (layer "F.Cu") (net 18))
 (segment (start 124.875305 82.45) (end 131.2 88.774695) (width 0.25) (layer "F.Cu") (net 18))
 (segment (start 125.7801 130.775) (end 124.6551 131.9) (width 0.25) (layer "F.Cu") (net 18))
 (via (at 131.9 122.7) (size 0.8) (drill 0.4) (layers "F.Cu" "B.Cu") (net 18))
 (via (at 131.9 100.6) (size 0.8) (drill 0.4) (layers "F.Cu" "B.Cu") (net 18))
 (segment (start 131.9 100.6) (end 131.9 122.7) (width 0.25) (layer "B.Cu") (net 18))
 (segment (start 125.848299 138.975) (end 130.49 138.975) (width 0.25) (layer "F.Cu") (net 14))
 (segment (start 115.45 134.125) (end 117.915 136.59) (width 0.25) (layer "F.Cu") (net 14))
 (segment (start 131.365 136.435) (end 132.54 135.26) (width 0.25) (layer "F.Cu") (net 14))
 (segment (start 116.559109 127.675) (end 115.45 128.784109) (width 0.25) (layer "F.Cu") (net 14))
 (segment (start 133.2575 82.9104) (end 134.3445 81.8234) (width 0.25) (layer "F.Cu") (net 14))
 (segment (start 123.463299 136.59) (end 125.848299 138.975) (width 0.25) (layer "F.Cu") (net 14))
 (segment (start 123.5201 127.675) (end 116.559109 127.675) (width 0.25) (layer "F.Cu") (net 14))
 (segment (start 120.8625 80.4625) (end 120.8625 77.4) (width 0.25) (layer "F.Cu") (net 14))
 (segment (start 134.3445 77.380149) (end 132.264351 75.3) (width 0.25) (layer "F.Cu") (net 14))
 (segment (start 115.45 128.784109) (end 115.45 134.125) (width 0.25) (layer "F.Cu") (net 14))
 (segment (start 131.365 138.1) (end 131.365 136.435) (width 0.25) (layer "F.Cu") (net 14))
 (segment (start 124.6451 128.8) (end 123.5201 127.675) (width 0.25) (layer "F.Cu") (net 14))
 (segment (start 134.3445 81.8234) (end 134.3445 77.380149) (width 0.25) (layer "F.Cu") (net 14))
 (segment (start 117.915 136.59) (end 123.463299 136.59) (width 0.25) (layer "F.Cu") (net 14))
 (segment (start 122.9625 75.3) (end 120.8625 77.4) (width 0.25) (layer "F.Cu") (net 14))
 (segment (start 130.49 138.975) (end 131.365 138.1) (width 0.25) (layer "F.Cu") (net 14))
 (segment (start 134.4551 133.3449) (end 134.4551 131.9) (width 0.25) (layer "F.Cu") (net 14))
 (segment (start 132.54 135.26) (end 134.4551 133.3449) (width 0.25) (layer "F.Cu") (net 14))
 (segment (start 132.264351 75.3) (end 122.9625 75.3) (width 0.25) (layer "F.Cu") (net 14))
 (via (at 120.8625 80.4625) (size 0.8) (drill 0.4) (layers "F.Cu" "B.Cu") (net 14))
 (segment (start 115.725 109.725) (end 115.725 82.375) (width 0.25) (layer "B.Cu") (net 14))
 (segment (start 115.725 82.375) (end 116.6426 81.4574) (width 0.25) (layer "B.Cu") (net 14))
 (segment (start 124.6451 128.8) (end 124.6451 118.6451) (width 0.25) (layer "B.Cu") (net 14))
 (segment (start 119.8676 81.4574) (end 120.8625 80.4625) (width 0.25) (layer "B.Cu") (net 14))
 (segment (start 124.6451 118.6451) (end 115.725 109.725) (width 0.25) (layer "B.Cu") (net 14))
 (segment (start 116.6426 81.4574) (end 119.8676 81.4574) (width 0.25) (layer "B.Cu") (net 14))
 (segment (start 119.3 95.2) (end 119.3 89.3329) (width 0.25) (layer "F.Cu") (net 16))
 (segment (start 130.975 120.749695) (end 130.975 104.896927) (width 0.25) (layer "F.Cu") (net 16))
 (segment (start 133.989109 130.775) (end 134.225 130.775) (width 0.25) (layer "F.Cu") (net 16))
 (segment (start 132.625 122.399695) (end 130.975 120.749695) (width 0.25) (layer "F.Cu") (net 16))
 (segment (start 133.989109 130.775) (end 134.921091 130.775) (width 0.25) (layer "F.Cu") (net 16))
 (segment (start 122.558467 95.9) (end 120 95.9) (width 0.25) (layer "F.Cu") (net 16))
 (segment (start 134.225 130.775) (end 135.5801 129.4199) (width 0.25) (layer "F.Cu") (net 16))
 (segment (start 135.5801 131.434009) (end 135.5801 134.7599) (width 0.25) (layer "F.Cu") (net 16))
 (segment (start 120 95.9) (end 119.3 95.2) (width 0.25) (layer "F.Cu") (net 16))
 (segment (start 135.5801 134.7599) (end 132.54 137.8) (width 0.25) (layer "F.Cu") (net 16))
 (segment (start 127.5101 131.225) (end 133.539109 131.225) (width 0.25) (layer "F.Cu") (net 16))
 (segment (start 134.921091 130.775) (end 135.5801 131.434009) (width 0.25) (layer "F.Cu") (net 16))
 (segment (start 126.8351 131.9) (end 127.5101 131.225) (width 0.25) (layer "F.Cu") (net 16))
 (segment (start 135.5801 129.4199) (end 135.5801 125.743704) (width 0.25) (layer "F.Cu") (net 16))
 (segment (start 119.3 89.3329) (end 117.9575 87.9904) (width 0.25) (layer "F.Cu") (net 16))
 (segment (start 133.539109 131.225) (end 133.989109 130.775) (width 0.25) (layer "F.Cu") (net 16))
 (segment (start 130.975 104.896927) (end 126.3103 100.232228) (width 0.25) (layer "F.Cu") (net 16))
 (segment (start 132.625 122.788604) (end 132.625 122.399695) (width 0.25) (layer "F.Cu") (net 16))
 (segment (start 135.5801 125.743704) (end 132.625 122.788604) (width 0.25) (layer "F.Cu") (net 16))
 (segment (start 126.3103 99.651833) (end 122.558467 95.9) (width 0.25) (layer "F.Cu") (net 16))
 (segment (start 126.3103 100.232228) (end 126.3103 99.651833) (width 0.25) (layer "F.Cu") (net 16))
 (segment (start 124.5 135.7) (end 124.5 134.6) (width 0.25) (layer "F.Cu") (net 15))
 (segment (start 116.95 134.05) (end 115.9 133) (width 0.25) (layer "F.Cu") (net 15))
 (segment (start 115.4 93.0879) (end 117.9575 90.5304) (width 0.25) (layer "F.Cu") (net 15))
 (segment (start 123.95 134.05) (end 116.95 134.05) (width 0.25) (layer "F.Cu") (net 15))
 (segment (start 125.2 136.4) (end 124.5 135.7) (width 0.25) (layer "F.Cu") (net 15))
 (segment (start 128.6 136.4) (end 125.2 136.4) (width 0.25) (layer "F.Cu") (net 15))
 (segment (start 115.9 129.9251) (end 117.0251 128.8) (width 0.25) (layer "F.Cu") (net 15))
 (segment (start 130 137.8) (end 128.6 136.4) (width 0.25) (layer "F.Cu") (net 15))
 (segment (start 117 123.2) (end 115.4 121.6) (width 0.25) (layer "F.Cu") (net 15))
 (segment (start 115.4 121.6) (end 115.4 93.0879) (width 0.25) (layer "F.Cu") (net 15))
 (segment (start 124.5 134.6) (end 123.95 134.05) (width 0.25) (layer "F.Cu") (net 15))
 (segment (start 115.9 133) (end 115.9 129.9251) (width 0.25) (layer "F.Cu") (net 15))
 (via (at 117 123.2) (size 0.8) (drill 0.4) (layers "F.Cu" "B.Cu") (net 15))
 (segment (start 117 123.2) (end 117.0251 123.2251) (width 0.25) (layer "B.Cu") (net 15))
 (segment (start 117.0251 123.2251) (end 117.0251 128.8) (width 0.25) (layer "B.Cu") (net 15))
 (segment (start 125.1375 77.4) (end 127.1 77.4) (width 0.25) (layer "F.Cu") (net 13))
 (segment (start 127.1 77.4) (end 130.2871 77.4) (width 0.25) (layer "F.Cu") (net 13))
 (segment (start 130.2871 77.4) (end 133.2575 80.3704) (width 0.25) (layer "F.Cu") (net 13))
 (via (at 127.1 77.4) (size 0.8) (drill 0.4) (layers "F.Cu" "B.Cu") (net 13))
 (segment (start 130.425 87.999695) (end 124.5 82.074695) (width 0.25) (layer "B.Cu") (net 13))
 (segment (start 130.9 92.3) (end 130.9 89.075305) (width 0.25) (layer "B.Cu") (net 13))
 (segment (start 130.9 89.075305) (end 130.425 88.600305) (width 0.25) (layer "B.Cu") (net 13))
 (segment (start 124.5 82.074695) (end 124.5 80) (width 0.25) (layer "B.Cu") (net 13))
 (segment (start 135.3975 96.7975) (end 130.9 92.3) (width 0.25) (layer "B.Cu") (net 13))
 (segment (start 135.3975 122.639158) (end 135.3975 96.7975) (width 0.25) (layer "B.Cu") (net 13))
 (segment (start 130.425 88.600305) (end 130.425 87.999695) (width 0.25) (layer "B.Cu") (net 13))
 (segment (start 130 128.036658) (end 135.3975 122.639158) (width 0.25) (layer "B.Cu") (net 13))
 (segment (start 130 135.26) (end 130 128.036658) (width 0.25) (layer "B.Cu") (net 13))
 (segment (start 124.5 80) (end 127.1 77.4) (width 0.25) (layer "B.Cu") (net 13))
 (segment (start 121.6 100.3) (end 119.55 102.35) (width 0.25) (layer "F.Cu") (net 3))
 (segment (start 119.55 118.15) (end 120 118.6) (width 0.25) (layer "F.Cu") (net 3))
 (segment (start 119.55 118.1) (end 119.55 118.15) (width 0.25) (layer "F.Cu") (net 3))
 (segment (start 119.55 102.35) (end 119.55 118.1) (width 0.25) (layer "F.Cu") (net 3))
 (via (at 120 118.6) (size 0.8) (drill 0.4) (layers "F.Cu" "B.Cu") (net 3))
 (via (at 121.6 100.3) (size 0.8) (drill 0.4) (layers "F.Cu" "B.Cu") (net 3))
 (segment (start 119.05 119.55) (end 119.05 135.075) (width 0.25) (layer "B.Cu") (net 3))
 (segment (start 123.125 98.775) (end 121.6 100.3) (width 0.25) (layer "B.Cu") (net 3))
 (segment (start 123.125 88.0779) (end 123.125 98.775) (width 0.25) (layer "B.Cu") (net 3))
 (segment (start 120 118.6) (end 119.05 119.55) (width 0.25) (layer "B.Cu") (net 3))
 (segment (start 117.9575 82.9104) (end 123.125 88.0779) (width 0.25) (layer "B.Cu") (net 3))
 (segment (start 119.05 135.075) (end 118.9 135.225) (width 0.25) (layer "B.Cu") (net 3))
 (segment (start 119.1 100.6) (end 119.1 118.1) (width 0.25) (layer "F.Cu") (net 4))
 (segment (start 119.1 118.1) (end 118.6 118.6) (width 0.25) (layer "F.Cu") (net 4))
 (segment (start 118.6 118.6) (end 118.7 118.5) (width 0.25) (layer "F.Cu") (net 4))
 (via (at 119.1 100.6) (size 0.8) (drill 0.4) (layers "F.Cu" "B.Cu") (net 4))
 (via (at 118.6 118.6) (size 0.8) (drill 0.4) (layers "F.Cu" "B.Cu") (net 4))
 (segment (start 118.9 137.765) (end 117.725 136.59) (width 0.25) (layer "B.Cu") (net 4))
 (segment (start 119.055 100.555) (end 119.055 97.159745) (width 0.25) (layer "B.Cu") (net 4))
 (segment (start 118.6 132.9) (end 118.6 118.6) (width 0.25) (layer "B.Cu") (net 4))
 (segment (start 119.1 100.6) (end 119.055 100.555) (width 0.25) (layer "B.Cu") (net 4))
 (segment (start 117.725 136.59) (end 117.725 133.775) (width 0.25) (layer "B.Cu") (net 4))
 (segment (start 119.055 97.159745) (end 116.5 94.604745) (width 0.25) (layer "B.Cu") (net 4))
 (segment (start 117.725 133.775) (end 118.6 132.9) (width 0.25) (layer "B.Cu") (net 4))
 (segment (start 116.5 94.604745) (end 116.5 86.9079) (width 0.25) (layer "B.Cu") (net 4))
 (segment (start 116.5 86.9079) (end 117.9575 85.4504) (width 0.25) (layer "B.Cu") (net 4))
 (segment (start 126.800001 82.600001) (end 128.7982 82.600001) (width 0.25) (layer "F.Cu") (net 6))
 (segment (start 126 81.8) (end 126.800001 82.600001) (width 0.25) (layer "F.Cu") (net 6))
 (via (at 126 81.8) (size 0.8) (drill 0.4) (layers "F.Cu" "B.Cu") (free) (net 6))
 (segment (start 130.875 87.813299) (end 130.875 87.9904) (width 0.25) (layer "B.Cu") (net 6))
 (segment (start 126 82.938299) (end 130.875 87.813299) (width 0.25) (layer "B.Cu") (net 6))
 (segment (start 126 81.8) (end 126 82.938299) (width 0.25) (layer "B.Cu") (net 6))
 (segment (start 130.875 87.9904) (end 133.2575 87.9904) (width 0.25) (layer "B.Cu") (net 6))
 (segment (start 126 80.6) (end 127.500002 82.100002) (width 0.25) (layer "F.Cu") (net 5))
 (segment (start 127.500002 82.100002) (end 128.7982 82.100002) (width 0.25) (layer "F.Cu") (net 5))
 (via (at 126 80.6) (size 0.8) (drill 0.4) (layers "F.Cu" "B.Cu") (free) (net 5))
 (segment (start 129.148497 85.4504) (end 133.2575 85.4504) (width 0.25) (layer "B.Cu") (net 5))
 (segment (start 126.725 81.325) (end 126.725 83.026903) (width 0.25) (layer "B.Cu") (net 5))
 (segment (start 126 80.6) (end 126.725 81.325) (width 0.25) (layer "B.Cu") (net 5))
 (segment (start 126.725 83.026903) (end 129.148497 85.4504) (width 0.25) (layer "B.Cu") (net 5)))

